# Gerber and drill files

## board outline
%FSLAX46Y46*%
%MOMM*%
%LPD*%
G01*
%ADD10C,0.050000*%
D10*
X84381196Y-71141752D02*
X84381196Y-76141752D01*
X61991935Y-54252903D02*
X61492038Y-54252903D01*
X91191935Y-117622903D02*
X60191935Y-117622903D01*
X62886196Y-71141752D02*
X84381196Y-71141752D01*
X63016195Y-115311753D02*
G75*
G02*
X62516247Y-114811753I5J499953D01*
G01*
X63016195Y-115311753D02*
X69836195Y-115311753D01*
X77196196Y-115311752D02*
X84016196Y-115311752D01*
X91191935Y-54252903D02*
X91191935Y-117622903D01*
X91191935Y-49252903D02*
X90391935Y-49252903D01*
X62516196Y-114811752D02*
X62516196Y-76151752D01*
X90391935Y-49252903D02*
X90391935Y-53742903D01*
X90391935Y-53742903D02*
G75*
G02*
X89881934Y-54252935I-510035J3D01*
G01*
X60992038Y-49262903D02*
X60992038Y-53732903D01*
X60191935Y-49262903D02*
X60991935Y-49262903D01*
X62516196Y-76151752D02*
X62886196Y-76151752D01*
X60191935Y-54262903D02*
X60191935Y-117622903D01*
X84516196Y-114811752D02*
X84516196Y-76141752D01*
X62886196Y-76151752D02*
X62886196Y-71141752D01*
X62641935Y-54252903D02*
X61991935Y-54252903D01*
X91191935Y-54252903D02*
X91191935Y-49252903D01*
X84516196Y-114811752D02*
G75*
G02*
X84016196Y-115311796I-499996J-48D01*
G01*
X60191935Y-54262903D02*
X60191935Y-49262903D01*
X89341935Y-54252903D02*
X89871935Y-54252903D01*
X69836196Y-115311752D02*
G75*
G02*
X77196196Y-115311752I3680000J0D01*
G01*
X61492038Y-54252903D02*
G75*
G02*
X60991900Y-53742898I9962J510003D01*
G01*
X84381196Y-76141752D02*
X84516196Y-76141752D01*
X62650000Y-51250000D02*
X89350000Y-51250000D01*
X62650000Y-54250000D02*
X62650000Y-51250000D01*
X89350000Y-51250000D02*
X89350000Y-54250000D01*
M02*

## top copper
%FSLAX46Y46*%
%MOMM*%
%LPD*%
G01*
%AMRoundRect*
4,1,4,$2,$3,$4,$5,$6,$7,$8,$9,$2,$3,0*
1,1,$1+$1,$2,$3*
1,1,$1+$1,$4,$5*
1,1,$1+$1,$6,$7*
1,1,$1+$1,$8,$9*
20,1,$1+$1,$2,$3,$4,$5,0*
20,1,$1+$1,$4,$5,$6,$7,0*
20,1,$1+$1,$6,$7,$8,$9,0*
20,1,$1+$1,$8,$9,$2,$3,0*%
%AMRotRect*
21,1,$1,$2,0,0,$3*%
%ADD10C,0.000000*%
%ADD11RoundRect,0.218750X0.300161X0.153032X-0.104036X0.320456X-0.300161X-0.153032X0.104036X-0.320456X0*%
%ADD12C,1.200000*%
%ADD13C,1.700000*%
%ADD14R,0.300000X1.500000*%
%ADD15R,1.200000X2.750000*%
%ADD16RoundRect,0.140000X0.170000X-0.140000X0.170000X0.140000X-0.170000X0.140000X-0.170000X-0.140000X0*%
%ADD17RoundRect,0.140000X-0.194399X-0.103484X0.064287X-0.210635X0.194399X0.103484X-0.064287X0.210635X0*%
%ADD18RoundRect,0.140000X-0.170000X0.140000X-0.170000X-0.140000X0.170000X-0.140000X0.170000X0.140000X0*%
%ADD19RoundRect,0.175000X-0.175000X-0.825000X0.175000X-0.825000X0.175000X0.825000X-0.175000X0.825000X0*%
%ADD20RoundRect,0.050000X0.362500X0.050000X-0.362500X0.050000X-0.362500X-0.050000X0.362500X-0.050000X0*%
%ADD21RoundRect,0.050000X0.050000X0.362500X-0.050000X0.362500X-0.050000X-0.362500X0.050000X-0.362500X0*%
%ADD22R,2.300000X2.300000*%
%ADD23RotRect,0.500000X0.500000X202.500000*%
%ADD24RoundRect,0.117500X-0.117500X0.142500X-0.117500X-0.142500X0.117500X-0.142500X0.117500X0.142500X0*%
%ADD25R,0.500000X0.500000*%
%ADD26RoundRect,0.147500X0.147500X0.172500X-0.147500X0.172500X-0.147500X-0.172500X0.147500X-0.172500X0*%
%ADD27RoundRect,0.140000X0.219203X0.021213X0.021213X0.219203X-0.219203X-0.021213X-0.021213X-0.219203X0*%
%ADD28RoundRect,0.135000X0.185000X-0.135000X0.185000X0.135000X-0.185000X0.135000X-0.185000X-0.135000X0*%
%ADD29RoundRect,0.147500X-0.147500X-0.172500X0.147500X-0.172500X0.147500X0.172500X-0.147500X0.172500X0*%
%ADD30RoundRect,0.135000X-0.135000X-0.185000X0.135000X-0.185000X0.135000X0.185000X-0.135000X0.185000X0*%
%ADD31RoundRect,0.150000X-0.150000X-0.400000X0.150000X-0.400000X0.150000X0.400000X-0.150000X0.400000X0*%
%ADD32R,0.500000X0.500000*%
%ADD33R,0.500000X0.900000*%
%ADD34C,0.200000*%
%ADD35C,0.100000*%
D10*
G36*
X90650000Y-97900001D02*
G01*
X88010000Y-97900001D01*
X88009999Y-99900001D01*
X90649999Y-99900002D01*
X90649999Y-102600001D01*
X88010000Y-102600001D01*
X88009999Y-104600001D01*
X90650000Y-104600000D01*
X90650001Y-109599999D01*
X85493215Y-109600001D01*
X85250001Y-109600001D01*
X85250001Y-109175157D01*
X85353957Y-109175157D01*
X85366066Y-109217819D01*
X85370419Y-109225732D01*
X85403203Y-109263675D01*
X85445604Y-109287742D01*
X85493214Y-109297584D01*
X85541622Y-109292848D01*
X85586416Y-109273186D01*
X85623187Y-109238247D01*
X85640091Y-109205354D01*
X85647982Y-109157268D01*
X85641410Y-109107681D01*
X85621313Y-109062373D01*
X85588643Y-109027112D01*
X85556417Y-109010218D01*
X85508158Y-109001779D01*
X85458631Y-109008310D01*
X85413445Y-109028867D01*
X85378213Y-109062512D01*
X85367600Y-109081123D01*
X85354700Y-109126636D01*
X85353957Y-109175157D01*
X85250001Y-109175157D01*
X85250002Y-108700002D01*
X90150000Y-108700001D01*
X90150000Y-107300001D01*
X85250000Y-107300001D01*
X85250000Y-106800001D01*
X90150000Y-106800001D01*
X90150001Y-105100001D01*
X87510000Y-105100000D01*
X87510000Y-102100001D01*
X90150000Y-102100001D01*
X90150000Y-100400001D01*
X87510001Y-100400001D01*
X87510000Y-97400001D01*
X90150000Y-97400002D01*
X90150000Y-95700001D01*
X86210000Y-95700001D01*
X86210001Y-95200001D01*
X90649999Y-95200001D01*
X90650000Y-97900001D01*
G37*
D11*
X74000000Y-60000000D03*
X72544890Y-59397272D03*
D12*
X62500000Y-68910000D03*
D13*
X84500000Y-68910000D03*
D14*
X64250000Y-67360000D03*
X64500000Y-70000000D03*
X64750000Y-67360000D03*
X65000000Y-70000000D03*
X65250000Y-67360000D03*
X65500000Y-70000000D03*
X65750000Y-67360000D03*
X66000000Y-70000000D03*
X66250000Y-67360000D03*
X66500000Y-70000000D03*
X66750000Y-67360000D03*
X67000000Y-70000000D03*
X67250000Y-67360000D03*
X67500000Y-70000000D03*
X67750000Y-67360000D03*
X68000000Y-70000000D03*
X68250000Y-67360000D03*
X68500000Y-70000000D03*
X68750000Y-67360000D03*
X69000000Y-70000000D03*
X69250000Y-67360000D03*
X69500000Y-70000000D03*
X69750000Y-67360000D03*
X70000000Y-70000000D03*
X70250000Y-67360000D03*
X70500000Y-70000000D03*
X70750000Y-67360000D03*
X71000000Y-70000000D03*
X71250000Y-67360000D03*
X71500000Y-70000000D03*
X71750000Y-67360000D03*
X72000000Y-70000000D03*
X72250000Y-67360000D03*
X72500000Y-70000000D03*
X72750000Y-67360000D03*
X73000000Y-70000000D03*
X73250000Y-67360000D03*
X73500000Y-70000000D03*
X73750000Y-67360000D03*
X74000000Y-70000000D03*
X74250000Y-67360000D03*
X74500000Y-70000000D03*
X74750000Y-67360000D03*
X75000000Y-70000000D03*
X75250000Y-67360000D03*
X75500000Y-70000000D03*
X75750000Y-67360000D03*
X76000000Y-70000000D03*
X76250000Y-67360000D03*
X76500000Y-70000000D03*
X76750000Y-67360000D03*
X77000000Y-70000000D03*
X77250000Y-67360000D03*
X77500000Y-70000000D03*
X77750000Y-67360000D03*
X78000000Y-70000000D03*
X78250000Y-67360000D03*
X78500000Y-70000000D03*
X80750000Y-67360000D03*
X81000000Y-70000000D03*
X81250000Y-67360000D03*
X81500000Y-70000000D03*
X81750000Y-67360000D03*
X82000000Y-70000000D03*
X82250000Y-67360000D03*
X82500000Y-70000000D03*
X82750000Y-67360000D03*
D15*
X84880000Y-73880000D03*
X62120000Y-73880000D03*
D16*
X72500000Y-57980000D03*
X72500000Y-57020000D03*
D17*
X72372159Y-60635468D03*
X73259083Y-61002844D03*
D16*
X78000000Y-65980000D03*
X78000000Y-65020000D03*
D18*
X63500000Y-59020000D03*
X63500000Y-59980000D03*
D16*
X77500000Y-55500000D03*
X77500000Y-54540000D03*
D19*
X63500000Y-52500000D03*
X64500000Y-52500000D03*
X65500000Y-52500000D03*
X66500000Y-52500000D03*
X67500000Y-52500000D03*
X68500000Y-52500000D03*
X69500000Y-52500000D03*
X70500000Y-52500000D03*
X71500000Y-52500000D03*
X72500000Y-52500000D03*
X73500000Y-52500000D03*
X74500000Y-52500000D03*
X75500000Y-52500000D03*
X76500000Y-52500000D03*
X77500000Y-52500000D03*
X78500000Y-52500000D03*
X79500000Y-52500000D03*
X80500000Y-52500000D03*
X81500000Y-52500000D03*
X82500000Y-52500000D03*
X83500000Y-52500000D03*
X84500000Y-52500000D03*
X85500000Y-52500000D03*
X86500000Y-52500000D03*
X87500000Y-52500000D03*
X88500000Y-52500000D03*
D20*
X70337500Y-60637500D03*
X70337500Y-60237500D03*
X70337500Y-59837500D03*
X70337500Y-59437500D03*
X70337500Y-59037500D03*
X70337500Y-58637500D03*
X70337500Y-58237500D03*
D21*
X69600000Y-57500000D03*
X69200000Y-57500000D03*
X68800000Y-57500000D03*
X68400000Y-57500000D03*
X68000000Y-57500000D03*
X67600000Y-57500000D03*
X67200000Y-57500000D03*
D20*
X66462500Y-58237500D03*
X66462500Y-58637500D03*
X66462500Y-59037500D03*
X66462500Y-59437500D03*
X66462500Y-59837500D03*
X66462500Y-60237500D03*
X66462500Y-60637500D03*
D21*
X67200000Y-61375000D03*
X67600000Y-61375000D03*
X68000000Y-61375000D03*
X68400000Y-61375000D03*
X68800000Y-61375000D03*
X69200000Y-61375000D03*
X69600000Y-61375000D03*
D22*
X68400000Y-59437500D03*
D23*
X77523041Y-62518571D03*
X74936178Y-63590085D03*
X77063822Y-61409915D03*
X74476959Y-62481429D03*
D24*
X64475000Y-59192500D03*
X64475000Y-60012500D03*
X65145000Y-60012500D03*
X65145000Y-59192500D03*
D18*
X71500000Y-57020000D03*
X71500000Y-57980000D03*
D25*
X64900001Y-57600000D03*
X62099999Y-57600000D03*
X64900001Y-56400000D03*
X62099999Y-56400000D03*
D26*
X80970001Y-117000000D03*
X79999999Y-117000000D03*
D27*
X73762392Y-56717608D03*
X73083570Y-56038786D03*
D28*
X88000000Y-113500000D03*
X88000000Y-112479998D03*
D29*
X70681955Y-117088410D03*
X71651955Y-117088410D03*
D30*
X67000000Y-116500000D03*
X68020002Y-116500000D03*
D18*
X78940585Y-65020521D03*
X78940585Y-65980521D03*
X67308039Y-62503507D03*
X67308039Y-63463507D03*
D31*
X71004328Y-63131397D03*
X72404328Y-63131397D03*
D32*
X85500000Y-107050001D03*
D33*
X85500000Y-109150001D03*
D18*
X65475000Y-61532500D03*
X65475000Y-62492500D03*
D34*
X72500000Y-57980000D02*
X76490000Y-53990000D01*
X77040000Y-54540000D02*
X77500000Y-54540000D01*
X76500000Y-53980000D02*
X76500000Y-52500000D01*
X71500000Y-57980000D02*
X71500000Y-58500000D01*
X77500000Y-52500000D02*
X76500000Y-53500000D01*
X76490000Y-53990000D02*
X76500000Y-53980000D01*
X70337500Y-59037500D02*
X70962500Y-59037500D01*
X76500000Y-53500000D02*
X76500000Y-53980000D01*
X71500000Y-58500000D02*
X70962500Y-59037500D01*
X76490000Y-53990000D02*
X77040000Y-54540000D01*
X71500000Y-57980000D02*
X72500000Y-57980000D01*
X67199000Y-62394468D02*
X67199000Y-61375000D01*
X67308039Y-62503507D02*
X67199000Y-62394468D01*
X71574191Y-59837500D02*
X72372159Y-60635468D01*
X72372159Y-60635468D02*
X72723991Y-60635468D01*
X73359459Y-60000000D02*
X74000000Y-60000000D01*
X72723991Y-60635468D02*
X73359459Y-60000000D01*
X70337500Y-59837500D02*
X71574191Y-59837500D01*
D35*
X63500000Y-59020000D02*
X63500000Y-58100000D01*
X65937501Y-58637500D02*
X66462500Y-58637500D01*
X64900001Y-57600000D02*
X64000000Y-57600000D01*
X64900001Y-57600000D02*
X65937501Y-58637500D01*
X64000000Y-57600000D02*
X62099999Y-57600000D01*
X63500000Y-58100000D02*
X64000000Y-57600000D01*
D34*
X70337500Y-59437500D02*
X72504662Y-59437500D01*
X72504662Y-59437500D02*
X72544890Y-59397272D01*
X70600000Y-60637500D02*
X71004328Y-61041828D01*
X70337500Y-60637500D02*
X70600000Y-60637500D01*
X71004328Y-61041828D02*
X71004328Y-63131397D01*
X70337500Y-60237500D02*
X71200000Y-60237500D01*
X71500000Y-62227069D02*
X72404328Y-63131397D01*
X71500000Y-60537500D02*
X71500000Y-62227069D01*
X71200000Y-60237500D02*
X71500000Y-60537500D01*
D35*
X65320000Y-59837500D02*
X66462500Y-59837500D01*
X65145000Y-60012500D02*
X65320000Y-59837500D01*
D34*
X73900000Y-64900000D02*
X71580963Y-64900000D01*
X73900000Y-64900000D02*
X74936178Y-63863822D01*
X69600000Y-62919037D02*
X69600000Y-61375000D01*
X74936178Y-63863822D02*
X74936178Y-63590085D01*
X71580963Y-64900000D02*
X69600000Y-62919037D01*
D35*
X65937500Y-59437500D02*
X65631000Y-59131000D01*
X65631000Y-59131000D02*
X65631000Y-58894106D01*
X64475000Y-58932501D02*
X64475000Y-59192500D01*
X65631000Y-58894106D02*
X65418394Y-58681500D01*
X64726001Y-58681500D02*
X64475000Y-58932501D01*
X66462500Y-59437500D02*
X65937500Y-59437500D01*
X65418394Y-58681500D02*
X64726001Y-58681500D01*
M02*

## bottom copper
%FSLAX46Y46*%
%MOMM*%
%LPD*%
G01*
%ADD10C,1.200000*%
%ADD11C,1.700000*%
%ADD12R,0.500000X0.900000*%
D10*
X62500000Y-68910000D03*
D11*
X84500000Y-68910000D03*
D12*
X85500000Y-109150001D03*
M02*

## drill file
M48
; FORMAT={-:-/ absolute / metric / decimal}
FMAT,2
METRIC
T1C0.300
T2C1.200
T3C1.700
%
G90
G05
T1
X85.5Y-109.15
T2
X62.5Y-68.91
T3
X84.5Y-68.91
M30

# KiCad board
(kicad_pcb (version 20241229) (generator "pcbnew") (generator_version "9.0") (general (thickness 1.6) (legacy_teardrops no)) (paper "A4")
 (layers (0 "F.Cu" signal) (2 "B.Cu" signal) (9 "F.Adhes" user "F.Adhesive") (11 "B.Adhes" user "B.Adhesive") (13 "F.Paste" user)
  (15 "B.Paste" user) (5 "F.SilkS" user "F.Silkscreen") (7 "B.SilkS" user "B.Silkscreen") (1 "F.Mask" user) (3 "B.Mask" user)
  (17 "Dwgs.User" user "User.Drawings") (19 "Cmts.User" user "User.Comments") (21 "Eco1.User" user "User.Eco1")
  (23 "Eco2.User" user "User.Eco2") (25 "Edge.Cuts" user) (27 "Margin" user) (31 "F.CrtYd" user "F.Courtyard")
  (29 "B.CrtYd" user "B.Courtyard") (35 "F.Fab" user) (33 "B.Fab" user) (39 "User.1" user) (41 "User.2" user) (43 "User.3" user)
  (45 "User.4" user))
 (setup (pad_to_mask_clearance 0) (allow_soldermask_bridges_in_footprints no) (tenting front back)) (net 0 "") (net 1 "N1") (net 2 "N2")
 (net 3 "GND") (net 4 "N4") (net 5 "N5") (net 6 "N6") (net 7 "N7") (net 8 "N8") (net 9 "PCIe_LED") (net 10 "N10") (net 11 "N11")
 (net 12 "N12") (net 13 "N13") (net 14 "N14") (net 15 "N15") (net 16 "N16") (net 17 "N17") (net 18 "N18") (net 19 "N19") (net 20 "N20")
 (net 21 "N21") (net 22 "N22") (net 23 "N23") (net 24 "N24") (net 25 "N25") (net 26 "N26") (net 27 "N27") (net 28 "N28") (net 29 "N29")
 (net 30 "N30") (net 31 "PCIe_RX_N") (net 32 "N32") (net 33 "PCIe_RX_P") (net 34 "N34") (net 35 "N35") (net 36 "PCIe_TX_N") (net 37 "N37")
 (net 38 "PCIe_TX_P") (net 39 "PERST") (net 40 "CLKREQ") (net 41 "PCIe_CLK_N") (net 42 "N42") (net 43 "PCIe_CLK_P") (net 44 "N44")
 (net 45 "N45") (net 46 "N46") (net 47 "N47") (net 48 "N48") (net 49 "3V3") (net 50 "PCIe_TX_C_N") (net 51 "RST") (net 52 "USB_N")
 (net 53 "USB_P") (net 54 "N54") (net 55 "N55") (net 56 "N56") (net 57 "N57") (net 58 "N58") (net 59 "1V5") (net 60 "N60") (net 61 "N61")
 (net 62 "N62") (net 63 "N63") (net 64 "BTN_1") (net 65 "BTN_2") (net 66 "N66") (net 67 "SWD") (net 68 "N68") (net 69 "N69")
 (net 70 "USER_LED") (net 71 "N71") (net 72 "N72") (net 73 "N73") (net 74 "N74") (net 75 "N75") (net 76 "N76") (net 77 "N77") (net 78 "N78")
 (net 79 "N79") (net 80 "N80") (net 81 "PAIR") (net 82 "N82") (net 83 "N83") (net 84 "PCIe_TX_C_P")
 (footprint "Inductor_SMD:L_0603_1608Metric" (layer "F.Cu") (at 73.272445 59.698636 157.5)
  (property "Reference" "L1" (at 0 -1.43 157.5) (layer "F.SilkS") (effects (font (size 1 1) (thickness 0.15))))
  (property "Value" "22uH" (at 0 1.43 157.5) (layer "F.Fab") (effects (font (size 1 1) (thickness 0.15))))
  (pad "1" smd roundrect (at -0.7875 -0.000001 157.5) (size 0.875 0.95) (layers "F.Cu" "F.Mask" "F.Paste") (roundrect_rratio 0.25)
   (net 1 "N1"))
  (pad "2" smd roundrect (at 0.7875 0.000001 157.5) (size 0.875 0.95) (layers "F.Cu" "F.Mask" "F.Paste") (roundrect_rratio 0.25)
   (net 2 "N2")))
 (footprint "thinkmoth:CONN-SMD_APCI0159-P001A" (layer "F.Cu") (at 73.5 70.62)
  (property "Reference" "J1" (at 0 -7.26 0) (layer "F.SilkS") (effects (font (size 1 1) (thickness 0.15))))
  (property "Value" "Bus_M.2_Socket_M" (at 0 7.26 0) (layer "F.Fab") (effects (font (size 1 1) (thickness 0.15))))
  (pad "" thru_hole circle (at -11 -1.71) (size 1.2 1.2) (drill 1.2) (layers "*.Cu" "*.Mask") (remove_unused_layers no))
  (pad "" thru_hole circle (at 11 -1.71) (size 1.7 1.7) (drill 1.7) (layers "*.Cu" "*.Mask") (remove_unused_layers no))
  (pad "1" smd rect (at -9.25 -3.26 90) (size 1.5 0.3) (layers "F.Cu" "F.Mask" "F.Paste") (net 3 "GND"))
  (pad "2" smd rect (at -9 -0.62 90) (size 1.5 0.3) (layers "F.Cu" "F.Mask" "F.Paste") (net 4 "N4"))
  (pad "3" smd rect (at -8.75 -3.26 90) (size 1.5 0.3) (layers "F.Cu" "F.Mask" "F.Paste") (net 3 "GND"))
  (pad "4" smd rect (at -8.5 -0.62 90) (size 1.5 0.3) (layers "F.Cu" "F.Mask" "F.Paste") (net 4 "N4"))
  (pad "5" smd rect (at -8.25 -3.26 90) (size 1.5 0.3) (layers "F.Cu" "F.Mask" "F.Paste") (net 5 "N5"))
  (pad "6" smd rect (at -8 -0.62 90) (size 1.5 0.3) (layers "F.Cu" "F.Mask" "F.Paste") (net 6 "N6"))
  (pad "7" smd rect (at -7.75 -3.26 90) (size 1.5 0.3) (layers "F.Cu" "F.Mask" "F.Paste") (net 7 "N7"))
  (pad "8" smd rect (at -7.5 -0.62 90) (size 1.5 0.3) (layers "F.Cu" "F.Mask" "F.Paste") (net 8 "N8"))
  (pad "9" smd rect (at -7.25 -3.26 90) (size 1.5 0.3) (layers "F.Cu" "F.Mask" "F.Paste") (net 3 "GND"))
  (pad "10" smd rect (at -7 -0.62 90) (size 1.5 0.3) (layers "F.Cu" "F.Mask" "F.Paste") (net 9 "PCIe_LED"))
  (pad "11" smd rect (at -6.75 -3.26 90) (size 1.5 0.3) (layers "F.Cu" "F.Mask" "F.Paste") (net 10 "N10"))
  (pad "12" smd rect (at -6.5 -0.62 90) (size 1.5 0.3) (layers "F.Cu" "F.Mask" "F.Paste") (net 4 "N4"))
  (pad "13" smd rect (at -6.25 -3.26 90) (size 1.5 0.3) (layers "F.Cu" "F.Mask" "F.Paste") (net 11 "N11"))
  (pad "14" smd rect (at -6 -0.62 90) (size 1.5 0.3) (layers "F.Cu" "F.Mask" "F.Paste") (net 4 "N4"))
  (pad "15" smd rect (at -5.75 -3.26 90) (size 1.5 0.3) (layers "F.Cu" "F.Mask" "F.Paste") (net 3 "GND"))
  (pad "16" smd rect (at -5.5 -0.62 90) (size 1.5 0.3) (layers "F.Cu" "F.Mask" "F.Paste") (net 4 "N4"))
  (pad "17" smd rect (at -5.25 -3.26 90) (size 1.5 0.3) (layers "F.Cu" "F.Mask" "F.Paste") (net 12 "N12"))
  (pad "18" smd rect (at -5 -0.62 90) (size 1.5 0.3) (layers "F.Cu" "F.Mask" "F.Paste") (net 4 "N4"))
  (pad "19" smd rect (at -4.75 -3.26 90) (size 1.5 0.3) (layers "F.Cu" "F.Mask" "F.Paste") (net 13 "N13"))
  (pad "20" smd rect (at -4.5 -0.62 90) (size 1.5 0.3) (layers "F.Cu" "F.Mask" "F.Paste") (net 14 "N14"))
  (pad "21" smd rect (at -4.25 -3.26 90) (size 1.5 0.3) (layers "F.Cu" "F.Mask" "F.Paste") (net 3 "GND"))
  (pad "22" smd rect (at -4 -0.62 90) (size 1.5 0.3) (layers "F.Cu" "F.Mask" "F.Paste") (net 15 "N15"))
  (pad "23" smd rect (at -3.75 -3.26 90) (size 1.5 0.3) (layers "F.Cu" "F.Mask" "F.Paste") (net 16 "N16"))
  (pad "24" smd rect (at -3.5 -0.62 90) (size 1.5 0.3) (layers "F.Cu" "F.Mask" "F.Paste") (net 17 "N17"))
  (pad "25" smd rect (at -3.25 -3.26 90) (size 1.5 0.3) (layers "F.Cu" "F.Mask" "F.Paste") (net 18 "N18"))
  (pad "26" smd rect (at -3 -0.62 90) (size 1.5 0.3) (layers "F.Cu" "F.Mask" "F.Paste") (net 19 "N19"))
  (pad "27" smd rect (at -2.75 -3.26 90) (size 1.5 0.3) (layers "F.Cu" "F.Mask" "F.Paste") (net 3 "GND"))
  (pad "28" smd rect (at -2.5 -0.62 90) (size 1.5 0.3) (layers "F.Cu" "F.Mask" "F.Paste") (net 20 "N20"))
  (pad "29" smd rect (at -2.25 -3.26 90) (size 1.5 0.3) (layers "F.Cu" "F.Mask" "F.Paste") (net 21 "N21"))
  (pad "30" smd rect (at -2 -0.62 90) (size 1.5 0.3) (layers "F.Cu" "F.Mask" "F.Paste") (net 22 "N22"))
  (pad "31" smd rect (at -1.75 -3.26 90) (size 1.5 0.3) (layers "F.Cu" "F.Mask" "F.Paste") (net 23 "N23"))
  (pad "32" smd rect (at -1.5 -0.62 90) (size 1.5 0.3) (layers "F.Cu" "F.Mask" "F.Paste") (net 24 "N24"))
  (pad "33" smd rect (at -1.25 -3.26 90) (size 1.5 0.3) (layers "F.Cu" "F.Mask" "F.Paste") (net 3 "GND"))
  (pad "34" smd rect (at -1 -0.62 90) (size 1.5 0.3) (layers "F.Cu" "F.Mask" "F.Paste") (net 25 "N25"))
  (pad "35" smd rect (at -0.75 -3.26 90) (size 1.5 0.3) (layers "F.Cu" "F.Mask" "F.Paste") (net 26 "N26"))
  (pad "36" smd rect (at -0.5 -0.62 90) (size 1.5 0.3) (layers "F.Cu" "F.Mask" "F.Paste") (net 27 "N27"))
  (pad "37" smd rect (at -0.25 -3.26 90) (size 1.5 0.3) (layers "F.Cu" "F.Mask" "F.Paste") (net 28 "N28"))
  (pad "38" smd rect (at 0 -0.62 90) (size 1.5 0.3) (layers "F.Cu" "F.Mask" "F.Paste") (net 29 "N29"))
  (pad "39" smd rect (at 0.25 -3.26 90) (size 1.5 0.3) (layers "F.Cu" "F.Mask" "F.Paste") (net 3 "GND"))
  (pad "40" smd rect (at 0.5 -0.62 90) (size 1.5 0.3) (layers "F.Cu" "F.Mask" "F.Paste") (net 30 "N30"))
  (pad "41" smd rect (at 0.75 -3.26 90) (size 1.5 0.3) (layers "F.Cu" "F.Mask" "F.Paste") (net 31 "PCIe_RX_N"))
  (pad "42" smd rect (at 1 -0.62 90) (size 1.5 0.3) (layers "F.Cu" "F.Mask" "F.Paste") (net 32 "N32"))
  (pad "43" smd rect (at 1.25 -3.26 90) (size 1.5 0.3) (layers "F.Cu" "F.Mask" "F.Paste") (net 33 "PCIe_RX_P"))
  (pad "44" smd rect (at 1.5 -0.62 90) (size 1.5 0.3) (layers "F.Cu" "F.Mask" "F.Paste") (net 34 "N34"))
  (pad "45" smd rect (at 1.75 -3.26 90) (size 1.5 0.3) (layers "F.Cu" "F.Mask" "F.Paste") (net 3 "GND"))
  (pad "46" smd rect (at 2 -0.62 90) (size 1.5 0.3) (layers "F.Cu" "F.Mask" "F.Paste") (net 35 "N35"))
  (pad "47" smd rect (at 2.25 -3.26 90) (size 1.5 0.3) (layers "F.Cu" "F.Mask" "F.Paste") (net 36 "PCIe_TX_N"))
  (pad "48" smd rect (at 2.5 -0.62 90) (size 1.5 0.3) (layers "F.Cu" "F.Mask" "F.Paste") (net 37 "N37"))
  (pad "49" smd rect (at 2.75 -3.26 90) (size 1.5 0.3) (layers "F.Cu" "F.Mask" "F.Paste") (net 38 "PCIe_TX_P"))
  (pad "50" smd rect (at 3 -0.62 90) (size 1.5 0.3) (layers "F.Cu" "F.Mask" "F.Paste") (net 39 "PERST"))
  (pad "51" smd rect (at 3.25 -3.26 90) (size 1.5 0.3) (layers "F.Cu" "F.Mask" "F.Paste") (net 3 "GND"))
  (pad "52" smd rect (at 3.5 -0.62 90) (size 1.5 0.3) (layers "F.Cu" "F.Mask" "F.Paste") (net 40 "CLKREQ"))
  (pad "53" smd rect (at 3.75 -3.26 90) (size 1.5 0.3) (layers "F.Cu" "F.Mask" "F.Paste") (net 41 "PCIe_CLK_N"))
  (pad "54" smd rect (at 4 -0.62 90) (size 1.5 0.3) (layers "F.Cu" "F.Mask" "F.Paste") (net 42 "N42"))
  (pad "55" smd rect (at 4.25 -3.26 90) (size 1.5 0.3) (layers "F.Cu" "F.Mask" "F.Paste") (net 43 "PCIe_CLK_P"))
  (pad "56" smd rect (at 4.5 -0.62 90) (size 1.5 0.3) (layers "F.Cu" "F.Mask" "F.Paste") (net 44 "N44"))
  (pad "57" smd rect (at 4.75 -3.26 90) (size 1.5 0.3) (layers "F.Cu" "F.Mask" "F.Paste") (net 3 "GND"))
  (pad "58" smd rect (at 5 -0.62 90) (size 1.5 0.3) (layers "F.Cu" "F.Mask" "F.Paste") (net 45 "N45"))
  (pad "67" smd rect (at 7.25 -3.26 90) (size 1.5 0.3) (layers "F.Cu" "F.Mask" "F.Paste") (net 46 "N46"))
  (pad "68" smd rect (at 7.5 -0.62 90) (size 1.5 0.3) (layers "F.Cu" "F.Mask" "F.Paste") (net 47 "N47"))
  (pad "69" smd rect (at 7.75 -3.26 90) (size 1.5 0.3) (layers "F.Cu" "F.Mask" "F.Paste") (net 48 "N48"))
  (pad "70" smd rect (at 8 -0.62 90) (size 1.5 0.3) (layers "F.Cu" "F.Mask" "F.Paste") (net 4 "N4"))
  (pad "71" smd rect (at 8.25 -3.26 90) (size 1.5 0.3) (layers "F.Cu" "F.Mask" "F.Paste") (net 3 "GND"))
  (pad "72" smd rect (at 8.5 -0.62 90) (size 1.5 0.3) (layers "F.Cu" "F.Mask" "F.Paste") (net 4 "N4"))
  (pad "73" smd rect (at 8.75 -3.26 90) (size 1.5 0.3) (layers "F.Cu" "F.Mask" "F.Paste") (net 3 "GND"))
  (pad "74" smd rect (at 9 -0.62 90) (size 1.5 0.3) (layers "F.Cu" "F.Mask" "F.Paste") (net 4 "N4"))
  (pad "75" smd rect (at 9.25 -3.26 90) (size 1.5 0.3) (layers "F.Cu" "F.Mask" "F.Paste") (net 3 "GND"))
  (pad "76" smd rect (at 11.38 3.26 90) (size 2.75 1.2) (layers "F.Cu" "F.Mask" "F.Paste"))
  (pad "77" smd rect (at -11.38 3.26 90) (size 2.75 1.2) (layers "F.Cu" "F.Mask" "F.Paste")))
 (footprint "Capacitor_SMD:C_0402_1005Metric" (layer "F.Cu") (at 72.5 57.5 90)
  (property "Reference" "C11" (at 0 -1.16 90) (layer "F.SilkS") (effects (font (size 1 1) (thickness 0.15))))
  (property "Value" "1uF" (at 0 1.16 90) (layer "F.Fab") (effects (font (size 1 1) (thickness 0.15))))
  (pad "1" smd roundrect (at -0.48 0 90) (size 0.56 0.62) (layers "F.Cu" "F.Mask" "F.Paste") (roundrect_rratio 0.25) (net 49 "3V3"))
  (pad "2" smd roundrect (at 0.48 0 90) (size 0.56 0.62) (layers "F.Cu" "F.Mask" "F.Paste") (roundrect_rratio 0.25) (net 3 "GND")))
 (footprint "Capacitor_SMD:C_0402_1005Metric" (layer "F.Cu") (at 72.815621 60.819156 -22.5)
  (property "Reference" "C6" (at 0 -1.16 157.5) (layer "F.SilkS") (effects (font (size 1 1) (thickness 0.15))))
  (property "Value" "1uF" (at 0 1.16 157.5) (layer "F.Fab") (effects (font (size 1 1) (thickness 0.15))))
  (pad "1" smd roundrect (at -0.48 0 337.5) (size 0.56 0.62) (layers "F.Cu" "F.Mask" "F.Paste") (roundrect_rratio 0.25) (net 1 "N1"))
  (pad "2" smd roundrect (at 0.48 0 337.5) (size 0.56 0.62) (layers "F.Cu" "F.Mask" "F.Paste") (roundrect_rratio 0.25) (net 3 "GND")))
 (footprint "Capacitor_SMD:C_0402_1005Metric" (layer "F.Cu") (at 78 65.5 90)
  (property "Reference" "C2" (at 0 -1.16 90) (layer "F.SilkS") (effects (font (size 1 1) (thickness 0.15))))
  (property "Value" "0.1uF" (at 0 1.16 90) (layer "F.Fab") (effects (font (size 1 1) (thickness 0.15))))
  (pad "1" smd roundrect (at -0.48 0 90) (size 0.56 0.62) (layers "F.Cu" "F.Mask" "F.Paste") (roundrect_rratio 0.25) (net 36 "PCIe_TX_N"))
  (pad "2" smd roundrect (at 0.48 0 90) (size 0.56 0.62) (layers "F.Cu" "F.Mask" "F.Paste") (roundrect_rratio 0.25) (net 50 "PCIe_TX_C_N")))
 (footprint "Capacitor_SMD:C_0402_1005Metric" (layer "F.Cu") (at 63.5 59.5 -90)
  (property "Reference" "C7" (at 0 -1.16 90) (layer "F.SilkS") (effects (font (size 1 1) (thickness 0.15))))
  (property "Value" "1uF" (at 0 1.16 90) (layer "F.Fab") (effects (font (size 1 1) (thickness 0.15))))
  (pad "1" smd roundrect (at -0.48 0 270) (size 0.56 0.62) (layers "F.Cu" "F.Mask" "F.Paste") (roundrect_rratio 0.25) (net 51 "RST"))
  (pad "2" smd roundrect (at 0.48 0 270) (size 0.56 0.62) (layers "F.Cu" "F.Mask" "F.Paste") (roundrect_rratio 0.25) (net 3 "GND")))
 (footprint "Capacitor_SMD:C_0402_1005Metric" (layer "F.Cu") (at 77.5 55.02 90)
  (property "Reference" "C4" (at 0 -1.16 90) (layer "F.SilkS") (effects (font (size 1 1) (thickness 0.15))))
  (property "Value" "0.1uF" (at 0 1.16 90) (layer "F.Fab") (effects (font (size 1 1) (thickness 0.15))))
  (pad "1" smd roundrect (at -0.48 0 90) (size 0.56 0.62) (layers "F.Cu" "F.Mask" "F.Paste") (roundrect_rratio 0.25) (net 3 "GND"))
  (pad "2" smd roundrect (at 0.48 0 90) (size 0.56 0.62) (layers "F.Cu" "F.Mask" "F.Paste") (roundrect_rratio 0.25) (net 49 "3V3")))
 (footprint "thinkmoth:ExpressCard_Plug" (layer "F.Cu") (at 76 52.5)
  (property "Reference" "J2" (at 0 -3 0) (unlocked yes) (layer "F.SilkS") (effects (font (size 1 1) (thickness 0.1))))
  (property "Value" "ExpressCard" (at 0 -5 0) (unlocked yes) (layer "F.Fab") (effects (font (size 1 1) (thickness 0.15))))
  (fp_line (start -13.35 -1.25) (end 13.35 -1.25) (stroke (width 0.05) (type default)) (layer "Edge.Cuts"))
  (fp_line (start -13.35 1.75) (end -13.35 -1.25) (stroke (width 0.05) (type default)) (layer "Edge.Cuts"))
  (fp_line (start 13.35 -1.25) (end 13.35 1.75) (stroke (width 0.05) (type default)) (layer "Edge.Cuts"))
  (pad "1" smd roundrect (at -12.5 0) (size 0.7 2) (layers "F.Cu" "F.Mask" "F.Paste") (roundrect_rratio 0.25) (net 3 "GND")
   (thermal_bridge_angle 45))
  (pad "2" smd roundrect (at -11.5 0) (size 0.7 2) (layers "F.Cu" "F.Mask" "F.Paste") (roundrect_rratio 0.25) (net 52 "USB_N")
   (thermal_bridge_angle 45))
  (pad "3" smd roundrect (at -10.5 0) (size 0.7 2) (layers "F.Cu" "F.Mask" "F.Paste") (roundrect_rratio 0.25) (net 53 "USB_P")
   (thermal_bridge_angle 45))
  (pad "4" smd roundrect (at -9.5 0) (size 0.7 2) (layers "F.Cu" "F.Mask" "F.Paste") (roundrect_rratio 0.25) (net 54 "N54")
   (thermal_bridge_angle 45))
  (pad "5" smd roundrect (at -8.5 0) (size 0.7 2) (layers "F.Cu" "F.Mask" "F.Paste") (roundrect_rratio 0.25) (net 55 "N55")
   (thermal_bridge_angle 45))
  (pad "6" smd roundrect (at -7.5 0) (size 0.7 2) (layers "F.Cu" "F.Mask" "F.Paste") (roundrect_rratio 0.25) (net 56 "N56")
   (thermal_bridge_angle 45))
  (pad "7" smd roundrect (at -6.5 0) (size 0.7 2) (layers "F.Cu" "F.Mask" "F.Paste") (roundrect_rratio 0.25) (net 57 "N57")
   (thermal_bridge_angle 45))
  (pad "8" smd roundrect (at -5.5 0) (size 0.7 2) (layers "F.Cu" "F.Mask" "F.Paste") (roundrect_rratio 0.25) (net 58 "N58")
   (thermal_bridge_angle 45))
  (pad "9" smd roundrect (at -4.5 0) (size 0.7 2) (layers "F.Cu" "F.Mask" "F.Paste") (roundrect_rratio 0.25) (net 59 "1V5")
   (thermal_bridge_angle 45))
  (pad "10" smd roundrect (at -3.5 0) (size 0.7 2) (layers "F.Cu" "F.Mask" "F.Paste") (roundrect_rratio 0.25) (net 59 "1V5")
   (thermal_bridge_angle 45))
  (pad "11" smd roundrect (at -2.5 0) (size 0.7 2) (layers "F.Cu" "F.Mask" "F.Paste") (roundrect_rratio 0.25) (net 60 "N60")
   (thermal_bridge_angle 45))
  (pad "12" smd roundrect (at -1.5 0) (size 0.7 2) (layers "F.Cu" "F.Mask" "F.Paste") (roundrect_rratio 0.25) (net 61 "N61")
   (thermal_bridge_angle 45))
  (pad "13" smd roundrect (at -0.5 0) (size 0.7 2) (layers "F.Cu" "F.Mask" "F.Paste") (roundrect_rratio 0.25) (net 39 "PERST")
   (thermal_bridge_angle 45))
  (pad "14" smd roundrect (at 0.5 0) (size 0.7 2) (layers "F.Cu" "F.Mask" "F.Paste") (roundrect_rratio 0.25) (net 49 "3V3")
   (thermal_bridge_angle 45))
  (pad "15" smd roundrect (at 1.5 0) (size 0.7 2) (layers "F.Cu" "F.Mask" "F.Paste") (roundrect_rratio 0.25) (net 49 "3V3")
   (thermal_bridge_angle 45))
  (pad "16" smd roundrect (at 2.5 0) (size 0.7 2) (layers "F.Cu" "F.Mask" "F.Paste") (roundrect_rratio 0.25) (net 40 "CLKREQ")
   (thermal_bridge_angle 45))
  (pad "17" smd roundrect (at 3.5 0) (size 0.7 2) (layers "F.Cu" "F.Mask" "F.Paste") (roundrect_rratio 0.25) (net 54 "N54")
   (thermal_bridge_angle 45))
  (pad "18" smd roundrect (at 4.5 0) (size 0.7 2) (layers "F.Cu" "F.Mask" "F.Paste") (roundrect_rratio 0.25) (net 41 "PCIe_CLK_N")
   (thermal_bridge_angle 45))
  (pad "19" smd roundrect (at 5.5 0) (size 0.7 2) (layers "F.Cu" "F.Mask" "F.Paste") (roundrect_rratio 0.25) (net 43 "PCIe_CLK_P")
   (thermal_bridge_angle 45))
  (pad "20" smd roundrect (at 6.5 0) (size 0.7 2) (layers "F.Cu" "F.Mask" "F.Paste") (roundrect_rratio 0.25) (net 3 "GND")
   (thermal_bridge_angle 45))
  (pad "21" smd roundrect (at 7.5 0) (size 0.7 2) (layers "F.Cu" "F.Mask" "F.Paste") (roundrect_rratio 0.25) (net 31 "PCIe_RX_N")
   (thermal_bridge_angle 45))
  (pad "22" smd roundrect (at 8.5 0) (size 0.7 2) (layers "F.Cu" "F.Mask" "F.Paste") (roundrect_rratio 0.25) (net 33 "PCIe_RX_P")
   (thermal_bridge_angle 45))
  (pad "23" smd roundrect (at 9.5 0) (size 0.7 2) (layers "F.Cu" "F.Mask" "F.Paste") (roundrect_rratio 0.25) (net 3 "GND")
   (thermal_bridge_angle 45))
  (pad "24" smd roundrect (at 10.5 0) (size 0.7 2) (layers "F.Cu" "F.Mask" "F.Paste") (roundrect_rratio 0.25) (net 36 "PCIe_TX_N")
   (thermal_bridge_angle 45))
  (pad "25" smd roundrect (at 11.5 0) (size 0.7 2) (layers "F.Cu" "F.Mask" "F.Paste") (roundrect_rratio 0.25) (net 38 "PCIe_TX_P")
   (thermal_bridge_angle 45))
  (pad "26" smd roundrect (at 12.5 0) (size 0.7 2) (layers "F.Cu" "F.Mask" "F.Paste") (roundrect_rratio 0.25) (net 3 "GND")
   (thermal_bridge_angle 45)))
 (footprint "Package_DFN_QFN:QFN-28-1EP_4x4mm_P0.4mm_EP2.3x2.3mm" (layer "F.Cu") (at 68.4 59.4375 180)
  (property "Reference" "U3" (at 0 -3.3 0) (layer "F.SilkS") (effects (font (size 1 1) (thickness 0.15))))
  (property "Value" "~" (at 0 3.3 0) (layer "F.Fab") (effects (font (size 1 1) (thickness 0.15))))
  (pad "" smd roundrect (at -0.575 -0.575 180) (size 0.93 0.93) (layers "F.Paste") (roundrect_rratio 0.25))
  (pad "" smd roundrect (at -0.575 0.575 180) (size 0.93 0.93) (layers "F.Paste") (roundrect_rratio 0.25))
  (pad "" smd roundrect (at 0.575 -0.575 180) (size 0.93 0.93) (layers "F.Paste") (roundrect_rratio 0.25))
  (pad "" smd roundrect (at 0.575 0.575 180) (size 0.93 0.93) (layers "F.Paste") (roundrect_rratio 0.25))
  (pad "1" smd roundrect (at -1.9375 -1.2 180) (size 0.825 0.2) (layers "F.Cu" "F.Mask" "F.Paste") (roundrect_rratio 0.25) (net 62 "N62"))
  (pad "2" smd roundrect (at -1.9375 -0.8 180) (size 0.825 0.2) (layers "F.Cu" "F.Mask" "F.Paste") (roundrect_rratio 0.25) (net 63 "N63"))
  (pad "3" smd roundrect (at -1.9375 -0.4 180) (size 0.825 0.2) (layers "F.Cu" "F.Mask" "F.Paste") (roundrect_rratio 0.25) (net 1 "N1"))
  (pad "4" smd roundrect (at -1.9375 0 180) (size 0.825 0.2) (layers "F.Cu" "F.Mask" "F.Paste") (roundrect_rratio 0.25) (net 2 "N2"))
  (pad "5" smd roundrect (at -1.9375 0.4 180) (size 0.825 0.2) (layers "F.Cu" "F.Mask" "F.Paste") (roundrect_rratio 0.25) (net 49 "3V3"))
  (pad "6" smd roundrect (at -1.9375 0.8 180) (size 0.825 0.2) (layers "F.Cu" "F.Mask" "F.Paste") (roundrect_rratio 0.25) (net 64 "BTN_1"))
  (pad "7" smd roundrect (at -1.9375 1.2 180) (size 0.825 0.2) (layers "F.Cu" "F.Mask" "F.Paste") (roundrect_rratio 0.25) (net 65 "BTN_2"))
  (pad "8" smd roundrect (at -1.2 1.9375 180) (size 0.2 0.825) (layers "F.Cu" "F.Mask" "F.Paste") (roundrect_rratio 0.25) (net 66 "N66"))
  (pad "9" smd roundrect (at -0.8 1.9375 180) (size 0.2 0.825) (layers "F.Cu" "F.Mask" "F.Paste") (roundrect_rratio 0.25) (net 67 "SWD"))
  (pad "10" smd roundrect (at -0.4 1.9375 180) (size 0.2 0.825) (layers "F.Cu" "F.Mask" "F.Paste") (roundrect_rratio 0.25) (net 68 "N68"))
  (pad "11" smd roundrect (at 0 1.9375 180) (size 0.2 0.825) (layers "F.Cu" "F.Mask" "F.Paste") (roundrect_rratio 0.25) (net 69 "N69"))
  (pad "12" smd roundrect (at 0.4 1.9375 180) (size 0.2 0.825) (layers "F.Cu" "F.Mask" "F.Paste") (roundrect_rratio 0.25) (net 52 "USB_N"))
  (pad "13" smd roundrect (at 0.8 1.9375 180) (size 0.2 0.825) (layers "F.Cu" "F.Mask" "F.Paste") (roundrect_rratio 0.25) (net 53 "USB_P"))
  (pad "14" smd roundrect (at 1.2 1.9375 180) (size 0.2 0.825) (layers "F.Cu" "F.Mask" "F.Paste") (roundrect_rratio 0.25)
   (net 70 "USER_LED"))
  (pad "15" smd roundrect (at 1.9375 1.2 180) (size 0.825 0.2) (layers "F.Cu" "F.Mask" "F.Paste") (roundrect_rratio 0.25) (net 9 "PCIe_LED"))
  (pad "16" smd roundrect (at 1.9375 0.8 180) (size 0.825 0.2) (layers "F.Cu" "F.Mask" "F.Paste") (roundrect_rratio 0.25) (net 51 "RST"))
  (pad "17" smd roundrect (at 1.9375 0.4 180) (size 0.825 0.2) (layers "F.Cu" "F.Mask" "F.Paste") (roundrect_rratio 0.25) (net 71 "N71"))
  (pad "18" smd roundrect (at 1.9375 0 180) (size 0.825 0.2) (layers "F.Cu" "F.Mask" "F.Paste") (roundrect_rratio 0.25) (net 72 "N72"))
  (pad "19" smd roundrect (at 1.9375 -0.4 180) (size 0.825 0.2) (layers "F.Cu" "F.Mask" "F.Paste") (roundrect_rratio 0.25) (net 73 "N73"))
  (pad "20" smd roundrect (at 1.9375 -0.8 180) (size 0.825 0.2) (layers "F.Cu" "F.Mask" "F.Paste") (roundrect_rratio 0.25) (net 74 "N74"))
  (pad "21" smd roundrect (at 1.9375 -1.2 180) (size 0.825 0.2) (layers "F.Cu" "F.Mask" "F.Paste") (roundrect_rratio 0.25) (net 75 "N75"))
  (pad "22" smd roundrect (at 1.2 -1.9375 180) (size 0.2 0.825) (layers "F.Cu" "F.Mask" "F.Paste") (roundrect_rratio 0.25) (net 1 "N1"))
  (pad "23" smd roundrect (at 0.8 -1.9375 180) (size 0.2 0.825) (layers "F.Cu" "F.Mask" "F.Paste") (roundrect_rratio 0.25) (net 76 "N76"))
  (pad "24" smd roundrect (at 0.4 -1.9375 180) (size 0.2 0.825) (layers "F.Cu" "F.Mask" "F.Paste") (roundrect_rratio 0.25) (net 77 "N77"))
  (pad "25" smd roundrect (at 0 -1.9375 180) (size 0.2 0.825) (layers "F.Cu" "F.Mask" "F.Paste") (roundrect_rratio 0.25) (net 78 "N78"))
  (pad "26" smd roundrect (at -0.4 -1.9375 180) (size 0.2 0.825) (layers "F.Cu" "F.Mask" "F.Paste") (roundrect_rratio 0.25) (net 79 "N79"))
  (pad "27" smd roundrect (at -0.8 -1.9375 180) (size 0.2 0.825) (layers "F.Cu" "F.Mask" "F.Paste") (roundrect_rratio 0.25) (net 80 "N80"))
  (pad "28" smd roundrect (at -1.2 -1.9375 180) (size 0.2 0.825) (layers "F.Cu" "F.Mask" "F.Paste") (roundrect_rratio 0.25) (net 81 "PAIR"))
  (pad "29" smd rect (at 0 0 180) (size 2.3 2.3) (layers "F.Cu" "F.Mask") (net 3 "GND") (zone_connect 2)))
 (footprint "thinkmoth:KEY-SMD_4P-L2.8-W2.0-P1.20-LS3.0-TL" (layer "F.Cu") (at 76 62.5 -157.5)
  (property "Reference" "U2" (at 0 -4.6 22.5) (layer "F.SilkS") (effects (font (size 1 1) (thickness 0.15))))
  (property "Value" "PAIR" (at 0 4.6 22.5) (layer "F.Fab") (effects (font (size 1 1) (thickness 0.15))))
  (pad "1" smd rect (at -1.4 -0.6 202.5) (size 0.5 0.5) (layers "F.Cu" "F.Mask" "F.Paste") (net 81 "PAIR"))
  (pad "2" smd rect (at 1.400001 -0.6 202.5) (size 0.5 0.5) (layers "F.Cu" "F.Mask" "F.Paste") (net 81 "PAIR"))
  (pad "3" smd rect (at -1.400001 0.6 202.5) (size 0.5 0.5) (layers "F.Cu" "F.Mask" "F.Paste") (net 3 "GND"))
  (pad "4" smd rect (at 1.4 0.6 202.5) (size 0.5 0.5) (layers "F.Cu" "F.Mask" "F.Paste") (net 3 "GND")))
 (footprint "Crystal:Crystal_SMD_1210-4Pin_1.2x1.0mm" (layer "F.Cu") (at 64.81 59.6025)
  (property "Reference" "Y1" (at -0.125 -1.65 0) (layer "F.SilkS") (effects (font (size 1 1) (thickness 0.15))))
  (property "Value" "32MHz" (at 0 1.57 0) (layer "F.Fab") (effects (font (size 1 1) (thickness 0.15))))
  (pad "1" smd roundrect (at -0.335 -0.41 270) (size 0.52 0.47) (layers "F.Cu" "F.Mask" "F.Paste") (roundrect_rratio 0.25) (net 72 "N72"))
  (pad "2" smd roundrect (at -0.335 0.41 270) (size 0.52 0.47) (layers "F.Cu" "F.Mask" "F.Paste") (roundrect_rratio 0.25) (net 3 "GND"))
  (pad "3" smd roundrect (at 0.335 0.41 270) (size 0.52 0.47) (layers "F.Cu" "F.Mask" "F.Paste") (roundrect_rratio 0.25) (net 73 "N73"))
  (pad "4" smd roundrect (at 0.335 -0.41 270) (size 0.52 0.47) (layers "F.Cu" "F.Mask" "F.Paste") (roundrect_rratio 0.25) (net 3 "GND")))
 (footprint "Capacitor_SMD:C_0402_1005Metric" (layer "F.Cu") (at 71.5 57.5 -90)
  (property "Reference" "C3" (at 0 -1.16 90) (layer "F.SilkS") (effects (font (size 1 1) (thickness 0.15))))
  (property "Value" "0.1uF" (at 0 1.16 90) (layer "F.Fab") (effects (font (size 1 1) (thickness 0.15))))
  (pad "1" smd roundrect (at -0.48 0 270) (size 0.56 0.62) (layers "F.Cu" "F.Mask" "F.Paste") (roundrect_rratio 0.25) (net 3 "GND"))
  (pad "2" smd roundrect (at 0.48 0 270) (size 0.56 0.62) (layers "F.Cu" "F.Mask" "F.Paste") (roundrect_rratio 0.25) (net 49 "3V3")))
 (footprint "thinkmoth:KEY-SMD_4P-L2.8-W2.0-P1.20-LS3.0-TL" (layer "F.Cu") (at 63.5 57 180)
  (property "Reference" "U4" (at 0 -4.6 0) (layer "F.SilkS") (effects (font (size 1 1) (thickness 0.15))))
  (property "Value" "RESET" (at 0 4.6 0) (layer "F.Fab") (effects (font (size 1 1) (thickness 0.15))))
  (pad "1" smd rect (at -1.400001 -0.6 180) (size 0.5 0.5) (layers "F.Cu" "F.Mask" "F.Paste") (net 51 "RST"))
  (pad "2" smd rect (at 1.400001 -0.6 180) (size 0.5 0.5) (layers "F.Cu" "F.Mask" "F.Paste") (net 51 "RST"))
  (pad "3" smd rect (at -1.400001 0.6 180) (size 0.5 0.5) (layers "F.Cu" "F.Mask" "F.Paste") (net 3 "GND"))
  (pad "4" smd rect (at 1.400001 0.6 180) (size 0.5 0.5) (layers "F.Cu" "F.Mask" "F.Paste") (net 3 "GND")))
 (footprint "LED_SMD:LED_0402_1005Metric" (layer "F.Cu") (at 80.485 117 180)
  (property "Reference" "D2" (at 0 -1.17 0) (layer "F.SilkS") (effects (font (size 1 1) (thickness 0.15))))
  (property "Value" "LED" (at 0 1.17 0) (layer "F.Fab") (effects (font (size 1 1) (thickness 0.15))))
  (pad "1" smd roundrect (at -0.485001 0 180) (size 0.59 0.64) (layers "F.Cu" "F.Mask" "F.Paste") (roundrect_rratio 0.25) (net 3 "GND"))
  (pad "2" smd roundrect (at 0.485001 0 180) (size 0.59 0.64) (layers "F.Cu" "F.Mask" "F.Paste") (roundrect_rratio 0.25) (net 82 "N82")))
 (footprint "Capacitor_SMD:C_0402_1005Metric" (layer "F.Cu") (at 73.422981 56.378197 135)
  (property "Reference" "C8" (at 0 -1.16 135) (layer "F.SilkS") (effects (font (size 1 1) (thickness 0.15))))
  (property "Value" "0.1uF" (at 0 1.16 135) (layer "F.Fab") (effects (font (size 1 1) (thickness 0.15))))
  (pad "1" smd roundrect (at -0.48 0 135) (size 0.56 0.62) (layers "F.Cu" "F.Mask" "F.Paste") (roundrect_rratio 0.25) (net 49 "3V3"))
  (pad "2" smd roundrect (at 0.48 0 135) (size 0.56 0.62) (layers "F.Cu" "F.Mask" "F.Paste") (roundrect_rratio 0.25) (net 3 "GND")))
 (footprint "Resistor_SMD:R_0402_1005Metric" (layer "F.Cu") (at 88 112.989999 90)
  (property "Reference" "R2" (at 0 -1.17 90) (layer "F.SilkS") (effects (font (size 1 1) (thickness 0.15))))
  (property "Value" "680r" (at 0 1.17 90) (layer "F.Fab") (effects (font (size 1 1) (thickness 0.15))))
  (pad "1" smd roundrect (at -0.510001 0 90) (size 0.54 0.64) (layers "F.Cu" "F.Mask" "F.Paste") (roundrect_rratio 0.25) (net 82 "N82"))
  (pad "2" smd roundrect (at 0.510001 0 90) (size 0.54 0.64) (layers "F.Cu" "F.Mask" "F.Paste") (roundrect_rratio 0.25) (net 70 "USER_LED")))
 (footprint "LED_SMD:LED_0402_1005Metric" (layer "F.Cu") (at 71.166955 117.08841)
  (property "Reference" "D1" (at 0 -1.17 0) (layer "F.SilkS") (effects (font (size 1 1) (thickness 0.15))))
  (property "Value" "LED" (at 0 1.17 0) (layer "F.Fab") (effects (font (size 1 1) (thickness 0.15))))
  (pad "1" smd roundrect (at -0.485 0) (size 0.59 0.64) (layers "F.Cu" "F.Mask" "F.Paste") (roundrect_rratio 0.25) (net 3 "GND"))
  (pad "2" smd roundrect (at 0.485 0) (size 0.59 0.64) (layers "F.Cu" "F.Mask" "F.Paste") (roundrect_rratio 0.25) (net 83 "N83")))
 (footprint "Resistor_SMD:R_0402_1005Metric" (layer "F.Cu") (at 67.510001 116.5)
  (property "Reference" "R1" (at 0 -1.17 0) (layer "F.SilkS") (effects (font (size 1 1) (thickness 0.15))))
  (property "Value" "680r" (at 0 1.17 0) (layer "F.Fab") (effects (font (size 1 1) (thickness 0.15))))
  (pad "1" smd roundrect (at -0.510001 0) (size 0.54 0.64) (layers "F.Cu" "F.Mask" "F.Paste") (roundrect_rratio 0.25) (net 83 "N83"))
  (pad "2" smd roundrect (at 0.510001 0) (size 0.54 0.64) (layers "F.Cu" "F.Mask" "F.Paste") (roundrect_rratio 0.25) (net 9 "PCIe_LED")))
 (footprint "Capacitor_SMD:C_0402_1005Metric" (layer "F.Cu") (at 78.940585 65.500521 -90)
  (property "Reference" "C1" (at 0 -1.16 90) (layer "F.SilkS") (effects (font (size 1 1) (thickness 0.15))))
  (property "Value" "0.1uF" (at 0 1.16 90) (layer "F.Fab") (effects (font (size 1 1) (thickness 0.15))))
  (pad "1" smd roundrect (at -0.48 0 270) (size 0.56 0.62) (layers "F.Cu" "F.Mask" "F.Paste") (roundrect_rratio 0.25) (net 38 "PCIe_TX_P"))
  (pad "2" smd roundrect (at 0.48 0 270) (size 0.56 0.62) (layers "F.Cu" "F.Mask" "F.Paste") (roundrect_rratio 0.25) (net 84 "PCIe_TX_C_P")))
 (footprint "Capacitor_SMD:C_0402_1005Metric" (layer "F.Cu") (at 67.308039 62.983507 -90)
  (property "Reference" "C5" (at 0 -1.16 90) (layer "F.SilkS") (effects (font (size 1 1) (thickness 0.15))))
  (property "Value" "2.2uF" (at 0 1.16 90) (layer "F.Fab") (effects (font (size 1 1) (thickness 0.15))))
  (pad "1" smd roundrect (at -0.48 0 270) (size 0.56 0.62) (layers "F.Cu" "F.Mask" "F.Paste") (roundrect_rratio 0.25) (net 1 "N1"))
  (pad "2" smd roundrect (at 0.48 0 270) (size 0.56 0.62) (layers "F.Cu" "F.Mask" "F.Paste") (roundrect_rratio 0.25) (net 3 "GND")))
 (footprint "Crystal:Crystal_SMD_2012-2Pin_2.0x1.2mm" (layer "F.Cu") (at 71.704328 63.131397)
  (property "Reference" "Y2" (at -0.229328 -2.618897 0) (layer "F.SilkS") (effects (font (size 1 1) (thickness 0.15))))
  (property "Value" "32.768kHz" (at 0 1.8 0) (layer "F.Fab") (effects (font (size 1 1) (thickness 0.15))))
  (pad "1" smd roundrect (at -0.7 0) (size 0.6 1.1) (layers "F.Cu" "F.Mask" "F.Paste") (roundrect_rratio 0.25) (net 62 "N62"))
  (pad "2" smd roundrect (at 0.7 0) (size 0.6 1.1) (layers "F.Cu" "F.Mask" "F.Paste") (roundrect_rratio 0.25) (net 63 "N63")))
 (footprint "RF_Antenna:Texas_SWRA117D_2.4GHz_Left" (layer "F.Cu") (at 85.5 107.050001 -90)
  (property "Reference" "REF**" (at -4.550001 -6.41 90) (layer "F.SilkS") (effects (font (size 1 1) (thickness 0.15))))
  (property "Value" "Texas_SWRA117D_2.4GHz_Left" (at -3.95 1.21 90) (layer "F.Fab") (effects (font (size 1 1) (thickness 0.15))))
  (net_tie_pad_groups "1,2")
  (fp_poly
   (pts (xy -2.45 -2.509999) (xy -4.45 -2.51) (xy -4.45 -5.149999) (xy -7.149999 -5.149999) (xy -7.15 -2.509999) (xy -9.15 -2.51)
    (xy -9.15 -5.15) (xy -11.85 -5.149999) (xy -11.85 -0.710001) (xy -11.35 -0.71) (xy -11.35 -4.65) (xy -9.649999 -4.65) (xy -9.65 -2.01)
    (xy -6.65 -2.010001) (xy -6.65 -4.65) (xy -4.95 -4.65) (xy -4.95 -2.01) (xy -1.950001 -2.01) (xy -1.95 -4.650001) (xy -0.25 -4.65)
    (xy -0.25 0.25) (xy 0.25 0.25) (xy 0.25 -4.65) (xy 1.65 -4.65) (xy 1.650001 0.249998) (xy 2.55 0.249999) (xy 2.55 0.006785)
    (xy 2.247583 0.006786) (xy 2.237741 0.054396) (xy 2.213674 0.096797) (xy 2.175731 0.129581) (xy 2.167818 0.133934)
    (xy 2.125156 0.146043) (xy 2.076635 0.1453) (xy 2.031122 0.1324) (xy 2.012511 0.121787) (xy 1.978866 0.086555) (xy 1.958309 0.041369)
    (xy 1.951778 -0.008158) (xy 1.960217 -0.056417) (xy 1.977111 -0.088643) (xy 2.012372 -0.121313) (xy 2.05768 -0.14141)
    (xy 2.107267 -0.147982) (xy 2.155353 -0.140091) (xy 2.188246 -0.123187) (xy 2.223185 -0.086416) (xy 2.242847 -0.041622)
    (xy 2.247583 0.006786) (xy 2.55 0.006785) (xy 2.549998 -5.150001) (xy -2.450001 -5.15) (xy -2.45 -2.509999))
   (stroke (width 0) (type solid)) (fill yes) (layer "F.Cu"))
  (pad "1" connect rect (at 0 0 270) (size 0.5 0.5) (layers "F.Cu"))
  (pad "2" thru_hole rect (at 2.1 0 270) (size 0.9 0.5) (drill 0.3) (layers "*.Cu") (remove_unused_layers no) (zone_connect 2)))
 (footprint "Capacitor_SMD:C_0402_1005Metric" (layer "F.Cu") (at 65.475 62.0125 -90)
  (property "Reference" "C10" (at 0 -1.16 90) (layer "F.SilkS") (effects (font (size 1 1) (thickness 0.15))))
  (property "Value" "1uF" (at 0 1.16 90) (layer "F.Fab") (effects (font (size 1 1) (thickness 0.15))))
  (pad "1" smd roundrect (at -0.48 0 270) (size 0.56 0.62) (layers "F.Cu" "F.Mask" "F.Paste") (roundrect_rratio 0.25) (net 74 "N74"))
  (pad "2" smd roundrect (at 0.48 0 270) (size 0.56 0.62) (layers "F.Cu" "F.Mask" "F.Paste") (roundrect_rratio 0.25) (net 3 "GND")))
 (gr_line (start 84.381196 71.141752) (end 84.381196 76.141752) (stroke (width 0.05) (type default)) (layer "Edge.Cuts"))
 (gr_line (start 61.991935 54.252903) (end 61.492038 54.252903) (stroke (width 0.05) (type default)) (layer "Edge.Cuts"))
 (gr_line (start 91.191935 117.622903) (end 60.191935 117.622903) (stroke (width 0.05) (type default)) (layer "Edge.Cuts"))
 (gr_line (start 62.886196 71.141752) (end 84.381196 71.141752) (stroke (width 0.05) (type default)) (layer "Edge.Cuts"))
 (gr_arc (start 63.016195 115.311753) (mid 62.662642 115.165306) (end 62.516195 114.811753) (stroke (width 0.05) (type default))
  (layer "Edge.Cuts"))
 (gr_line (start 63.016195 115.311753) (end 69.836195 115.311753) (stroke (width 0.05) (type default)) (layer "Edge.Cuts"))
 (gr_line (start 77.196196 115.311752) (end 84.016196 115.311752) (stroke (width 0.05) (type default)) (layer "Edge.Cuts"))
 (gr_line (start 91.191935 54.252903) (end 91.191935 117.622903) (stroke (width 0.05) (type default)) (layer "Edge.Cuts"))
 (gr_line (start 91.191935 49.252903) (end 90.391935 49.252903) (stroke (width 0.05) (type default)) (layer "Edge.Cuts"))
 (gr_line (start 62.516196 114.811752) (end 62.516196 76.151752) (stroke (width 0.05) (type default)) (layer "Edge.Cuts"))
 (gr_line (start 90.391935 49.252903) (end 90.391935 53.742903) (stroke (width 0.05) (type default)) (layer "Edge.Cuts"))
 (gr_arc (start 90.391935 53.742903) (mid 90.242559 54.103528) (end 89.881934 54.252908) (stroke (width 0.05) (type default))
  (layer "Edge.Cuts"))
 (gr_line (start 60.992038 49.262903) (end 60.992038 53.732903) (stroke (width 0.05) (type default)) (layer "Edge.Cuts"))
 (gr_line (start 60.191935 49.262903) (end 60.991935 49.262903) (stroke (width 0.05) (type default)) (layer "Edge.Cuts"))
 (gr_line (start 62.516196 76.151752) (end 62.886196 76.151752) (stroke (width 0.05) (type default)) (layer "Edge.Cuts"))
 (gr_line (start 60.191935 54.262903) (end 60.191935 117.622903) (stroke (width 0.05) (type default)) (layer "Edge.Cuts"))
 (gr_line (start 84.516196 114.811752) (end 84.516196 76.141752) (stroke (width 0.05) (type default)) (layer "Edge.Cuts"))
 (gr_line (start 62.886196 76.151752) (end 62.886196 71.141752) (stroke (width 0.05) (type default)) (layer "Edge.Cuts"))
 (gr_line (start 62.641935 54.252903) (end 61.991935 54.252903) (stroke (width 0.05) (type default)) (layer "Edge.Cuts"))
 (gr_line (start 91.191935 54.252903) (end 91.191935 49.252903) (stroke (width 0.05) (type default)) (layer "Edge.Cuts"))
 (gr_arc (start 84.516196 114.811752) (mid 84.369749 115.165305) (end 84.016196 115.311752) (stroke (width 0.05) (type default))
  (layer "Edge.Cuts"))
 (gr_line (start 60.191935 54.262903) (end 60.191935 49.262903) (stroke (width 0.05) (type default)) (layer "Edge.Cuts"))
 (gr_line (start 89.341935 54.252903) (end 89.871935 54.252903) (stroke (width 0.05) (type default)) (layer "Edge.Cuts"))
 (gr_arc (start 69.836196 115.311752) (mid 73.516196 111.631752) (end 77.196196 115.311752) (stroke (width 0.05) (type default))
  (layer "Edge.Cuts"))
 (gr_arc (start 61.492038 54.252903) (mid 61.137822 54.100042) (end 60.991935 53.742898) (stroke (width 0.05) (type default))
  (layer "Edge.Cuts"))
 (gr_line (start 84.381196 76.141752) (end 84.516196 76.141752) (stroke (width 0.05) (type default)) (layer "Edge.Cuts"))
 (segment (start 72.5 57.98) (end 76.49 53.99) (width 0.2) (layer "F.Cu") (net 49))
 (segment (start 77.04 54.54) (end 77.5 54.54) (width 0.2) (layer "F.Cu") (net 49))
 (segment (start 76.5 53.98) (end 76.5 52.5) (width 0.2) (layer "F.Cu") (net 49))
 (segment (start 71.5 57.98) (end 71.5 58.5) (width 0.2) (layer "F.Cu") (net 49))
 (segment (start 77.5 52.5) (end 76.5 53.5) (width 0.2) (layer "F.Cu") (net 49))
 (segment (start 76.49 53.99) (end 76.5 53.98) (width 0.2) (layer "F.Cu") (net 49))
 (segment (start 70.3375 59.0375) (end 70.9625 59.0375) (width 0.2) (layer "F.Cu") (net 49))
 (segment (start 76.5 53.5) (end 76.5 53.98) (width 0.2) (layer "F.Cu") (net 49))
 (segment (start 71.5 58.5) (end 70.9625 59.0375) (width 0.2) (layer "F.Cu") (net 49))
 (segment (start 76.49 53.99) (end 77.04 54.54) (width 0.2) (layer "F.Cu") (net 49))
 (segment (start 71.5 57.98) (end 72.5 57.98) (width 0.2) (layer "F.Cu") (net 49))
 (segment (start 67.199 62.394468) (end 67.199 61.375) (width 0.2) (layer "F.Cu") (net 1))
 (segment (start 67.308039 62.503507) (end 67.199 62.394468) (width 0.2) (layer "F.Cu") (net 1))
 (segment (start 71.574191 59.8375) (end 72.372159 60.635468) (width 0.2) (layer "F.Cu") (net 1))
 (segment (start 72.372159 60.635468) (end 72.723991 60.635468) (width 0.2) (layer "F.Cu") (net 1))
 (segment (start 73.359459 60) (end 74 60) (width 0.2) (layer "F.Cu") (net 1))
 (segment (start 72.723991 60.635468) (end 73.359459 60) (width 0.2) (layer "F.Cu") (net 1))
 (segment (start 70.3375 59.8375) (end 71.574191 59.8375) (width 0.2) (layer "F.Cu") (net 1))
 (segment (start 63.5 59.02) (end 63.5 58.1) (width 0.1) (layer "F.Cu") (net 51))
 (segment (start 65.937501 58.6375) (end 66.4625 58.6375) (width 0.1) (layer "F.Cu") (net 51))
 (segment (start 64.900001 57.6) (end 64 57.6) (width 0.1) (layer "F.Cu") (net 51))
 (segment (start 64.900001 57.6) (end 65.937501 58.6375) (width 0.1) (layer "F.Cu") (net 51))
 (segment (start 64 57.6) (end 62.099999 57.6) (width 0.1) (layer "F.Cu") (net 51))
 (segment (start 63.5 58.1) (end 64 57.6) (width 0.1) (layer "F.Cu") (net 51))
 (segment (start 70.3375 59.4375) (end 72.504662 59.4375) (width 0.2) (layer "F.Cu") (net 2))
 (segment (start 72.504662 59.4375) (end 72.54489 59.397272) (width 0.2) (layer "F.Cu") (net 2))
 (segment (start 70.6 60.6375) (end 71.004328 61.041828) (width 0.2) (layer "F.Cu") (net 62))
 (segment (start 70.3375 60.6375) (end 70.6 60.6375) (width 0.2) (layer "F.Cu") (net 62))
 (segment (start 71.004328 61.041828) (end 71.004328 63.131397) (width 0.2) (layer "F.Cu") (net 62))
 (segment (start 70.3375 60.2375) (end 71.2 60.2375) (width 0.2) (layer "F.Cu") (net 63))
 (segment (start 71.5 62.227069) (end 72.404328 63.131397) (width 0.2) (layer "F.Cu") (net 63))
 (segment (start 71.5 60.5375) (end 71.5 62.227069) (width 0.2) (layer "F.Cu") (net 63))
 (segment (start 71.2 60.2375) (end 71.5 60.5375) (width 0.2) (layer "F.Cu") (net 63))
 (segment (start 65.32 59.8375) (end 66.4625 59.8375) (width 0.1) (layer "F.Cu") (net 73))
 (segment (start 65.145 60.0125) (end 65.32 59.8375) (width 0.1) (layer "F.Cu") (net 73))
 (segment (start 73.9 64.9) (end 71.580963 64.9) (width 0.2) (layer "F.Cu") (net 81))
 (segment (start 73.9 64.9) (end 74.936178 63.863822) (width 0.2) (layer "F.Cu") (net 81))
 (segment (start 69.6 62.919037) (end 69.6 61.375) (width 0.2) (layer "F.Cu") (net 81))
 (segment (start 74.936178 63.863822) (end 74.936178 63.590085) (width 0.2) (layer "F.Cu") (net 81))
 (segment (start 71.580963 64.9) (end 69.6 62.919037) (width 0.2) (layer "F.Cu") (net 81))
 (segment (start 65.9375 59.4375) (end 65.631 59.131) (width 0.1) (layer "F.Cu") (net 72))
 (segment (start 65.631 59.131) (end 65.631 58.894106) (width 0.1) (layer "F.Cu") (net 72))
 (segment (start 64.475 58.932501) (end 64.475 59.1925) (width 0.1) (layer "F.Cu") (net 72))
 (segment (start 65.631 58.894106) (end 65.418394 58.6815) (width 0.1) (layer "F.Cu") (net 72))
 (segment (start 64.726001 58.6815) (end 64.475 58.932501) (width 0.1) (layer "F.Cu") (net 72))
 (segment (start 66.4625 59.4375) (end 65.9375 59.4375) (width 0.1) (layer "F.Cu") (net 72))
 (segment (start 65.418394 58.6815) (end 64.726001 58.6815) (width 0.1) (layer "F.Cu") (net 72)))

